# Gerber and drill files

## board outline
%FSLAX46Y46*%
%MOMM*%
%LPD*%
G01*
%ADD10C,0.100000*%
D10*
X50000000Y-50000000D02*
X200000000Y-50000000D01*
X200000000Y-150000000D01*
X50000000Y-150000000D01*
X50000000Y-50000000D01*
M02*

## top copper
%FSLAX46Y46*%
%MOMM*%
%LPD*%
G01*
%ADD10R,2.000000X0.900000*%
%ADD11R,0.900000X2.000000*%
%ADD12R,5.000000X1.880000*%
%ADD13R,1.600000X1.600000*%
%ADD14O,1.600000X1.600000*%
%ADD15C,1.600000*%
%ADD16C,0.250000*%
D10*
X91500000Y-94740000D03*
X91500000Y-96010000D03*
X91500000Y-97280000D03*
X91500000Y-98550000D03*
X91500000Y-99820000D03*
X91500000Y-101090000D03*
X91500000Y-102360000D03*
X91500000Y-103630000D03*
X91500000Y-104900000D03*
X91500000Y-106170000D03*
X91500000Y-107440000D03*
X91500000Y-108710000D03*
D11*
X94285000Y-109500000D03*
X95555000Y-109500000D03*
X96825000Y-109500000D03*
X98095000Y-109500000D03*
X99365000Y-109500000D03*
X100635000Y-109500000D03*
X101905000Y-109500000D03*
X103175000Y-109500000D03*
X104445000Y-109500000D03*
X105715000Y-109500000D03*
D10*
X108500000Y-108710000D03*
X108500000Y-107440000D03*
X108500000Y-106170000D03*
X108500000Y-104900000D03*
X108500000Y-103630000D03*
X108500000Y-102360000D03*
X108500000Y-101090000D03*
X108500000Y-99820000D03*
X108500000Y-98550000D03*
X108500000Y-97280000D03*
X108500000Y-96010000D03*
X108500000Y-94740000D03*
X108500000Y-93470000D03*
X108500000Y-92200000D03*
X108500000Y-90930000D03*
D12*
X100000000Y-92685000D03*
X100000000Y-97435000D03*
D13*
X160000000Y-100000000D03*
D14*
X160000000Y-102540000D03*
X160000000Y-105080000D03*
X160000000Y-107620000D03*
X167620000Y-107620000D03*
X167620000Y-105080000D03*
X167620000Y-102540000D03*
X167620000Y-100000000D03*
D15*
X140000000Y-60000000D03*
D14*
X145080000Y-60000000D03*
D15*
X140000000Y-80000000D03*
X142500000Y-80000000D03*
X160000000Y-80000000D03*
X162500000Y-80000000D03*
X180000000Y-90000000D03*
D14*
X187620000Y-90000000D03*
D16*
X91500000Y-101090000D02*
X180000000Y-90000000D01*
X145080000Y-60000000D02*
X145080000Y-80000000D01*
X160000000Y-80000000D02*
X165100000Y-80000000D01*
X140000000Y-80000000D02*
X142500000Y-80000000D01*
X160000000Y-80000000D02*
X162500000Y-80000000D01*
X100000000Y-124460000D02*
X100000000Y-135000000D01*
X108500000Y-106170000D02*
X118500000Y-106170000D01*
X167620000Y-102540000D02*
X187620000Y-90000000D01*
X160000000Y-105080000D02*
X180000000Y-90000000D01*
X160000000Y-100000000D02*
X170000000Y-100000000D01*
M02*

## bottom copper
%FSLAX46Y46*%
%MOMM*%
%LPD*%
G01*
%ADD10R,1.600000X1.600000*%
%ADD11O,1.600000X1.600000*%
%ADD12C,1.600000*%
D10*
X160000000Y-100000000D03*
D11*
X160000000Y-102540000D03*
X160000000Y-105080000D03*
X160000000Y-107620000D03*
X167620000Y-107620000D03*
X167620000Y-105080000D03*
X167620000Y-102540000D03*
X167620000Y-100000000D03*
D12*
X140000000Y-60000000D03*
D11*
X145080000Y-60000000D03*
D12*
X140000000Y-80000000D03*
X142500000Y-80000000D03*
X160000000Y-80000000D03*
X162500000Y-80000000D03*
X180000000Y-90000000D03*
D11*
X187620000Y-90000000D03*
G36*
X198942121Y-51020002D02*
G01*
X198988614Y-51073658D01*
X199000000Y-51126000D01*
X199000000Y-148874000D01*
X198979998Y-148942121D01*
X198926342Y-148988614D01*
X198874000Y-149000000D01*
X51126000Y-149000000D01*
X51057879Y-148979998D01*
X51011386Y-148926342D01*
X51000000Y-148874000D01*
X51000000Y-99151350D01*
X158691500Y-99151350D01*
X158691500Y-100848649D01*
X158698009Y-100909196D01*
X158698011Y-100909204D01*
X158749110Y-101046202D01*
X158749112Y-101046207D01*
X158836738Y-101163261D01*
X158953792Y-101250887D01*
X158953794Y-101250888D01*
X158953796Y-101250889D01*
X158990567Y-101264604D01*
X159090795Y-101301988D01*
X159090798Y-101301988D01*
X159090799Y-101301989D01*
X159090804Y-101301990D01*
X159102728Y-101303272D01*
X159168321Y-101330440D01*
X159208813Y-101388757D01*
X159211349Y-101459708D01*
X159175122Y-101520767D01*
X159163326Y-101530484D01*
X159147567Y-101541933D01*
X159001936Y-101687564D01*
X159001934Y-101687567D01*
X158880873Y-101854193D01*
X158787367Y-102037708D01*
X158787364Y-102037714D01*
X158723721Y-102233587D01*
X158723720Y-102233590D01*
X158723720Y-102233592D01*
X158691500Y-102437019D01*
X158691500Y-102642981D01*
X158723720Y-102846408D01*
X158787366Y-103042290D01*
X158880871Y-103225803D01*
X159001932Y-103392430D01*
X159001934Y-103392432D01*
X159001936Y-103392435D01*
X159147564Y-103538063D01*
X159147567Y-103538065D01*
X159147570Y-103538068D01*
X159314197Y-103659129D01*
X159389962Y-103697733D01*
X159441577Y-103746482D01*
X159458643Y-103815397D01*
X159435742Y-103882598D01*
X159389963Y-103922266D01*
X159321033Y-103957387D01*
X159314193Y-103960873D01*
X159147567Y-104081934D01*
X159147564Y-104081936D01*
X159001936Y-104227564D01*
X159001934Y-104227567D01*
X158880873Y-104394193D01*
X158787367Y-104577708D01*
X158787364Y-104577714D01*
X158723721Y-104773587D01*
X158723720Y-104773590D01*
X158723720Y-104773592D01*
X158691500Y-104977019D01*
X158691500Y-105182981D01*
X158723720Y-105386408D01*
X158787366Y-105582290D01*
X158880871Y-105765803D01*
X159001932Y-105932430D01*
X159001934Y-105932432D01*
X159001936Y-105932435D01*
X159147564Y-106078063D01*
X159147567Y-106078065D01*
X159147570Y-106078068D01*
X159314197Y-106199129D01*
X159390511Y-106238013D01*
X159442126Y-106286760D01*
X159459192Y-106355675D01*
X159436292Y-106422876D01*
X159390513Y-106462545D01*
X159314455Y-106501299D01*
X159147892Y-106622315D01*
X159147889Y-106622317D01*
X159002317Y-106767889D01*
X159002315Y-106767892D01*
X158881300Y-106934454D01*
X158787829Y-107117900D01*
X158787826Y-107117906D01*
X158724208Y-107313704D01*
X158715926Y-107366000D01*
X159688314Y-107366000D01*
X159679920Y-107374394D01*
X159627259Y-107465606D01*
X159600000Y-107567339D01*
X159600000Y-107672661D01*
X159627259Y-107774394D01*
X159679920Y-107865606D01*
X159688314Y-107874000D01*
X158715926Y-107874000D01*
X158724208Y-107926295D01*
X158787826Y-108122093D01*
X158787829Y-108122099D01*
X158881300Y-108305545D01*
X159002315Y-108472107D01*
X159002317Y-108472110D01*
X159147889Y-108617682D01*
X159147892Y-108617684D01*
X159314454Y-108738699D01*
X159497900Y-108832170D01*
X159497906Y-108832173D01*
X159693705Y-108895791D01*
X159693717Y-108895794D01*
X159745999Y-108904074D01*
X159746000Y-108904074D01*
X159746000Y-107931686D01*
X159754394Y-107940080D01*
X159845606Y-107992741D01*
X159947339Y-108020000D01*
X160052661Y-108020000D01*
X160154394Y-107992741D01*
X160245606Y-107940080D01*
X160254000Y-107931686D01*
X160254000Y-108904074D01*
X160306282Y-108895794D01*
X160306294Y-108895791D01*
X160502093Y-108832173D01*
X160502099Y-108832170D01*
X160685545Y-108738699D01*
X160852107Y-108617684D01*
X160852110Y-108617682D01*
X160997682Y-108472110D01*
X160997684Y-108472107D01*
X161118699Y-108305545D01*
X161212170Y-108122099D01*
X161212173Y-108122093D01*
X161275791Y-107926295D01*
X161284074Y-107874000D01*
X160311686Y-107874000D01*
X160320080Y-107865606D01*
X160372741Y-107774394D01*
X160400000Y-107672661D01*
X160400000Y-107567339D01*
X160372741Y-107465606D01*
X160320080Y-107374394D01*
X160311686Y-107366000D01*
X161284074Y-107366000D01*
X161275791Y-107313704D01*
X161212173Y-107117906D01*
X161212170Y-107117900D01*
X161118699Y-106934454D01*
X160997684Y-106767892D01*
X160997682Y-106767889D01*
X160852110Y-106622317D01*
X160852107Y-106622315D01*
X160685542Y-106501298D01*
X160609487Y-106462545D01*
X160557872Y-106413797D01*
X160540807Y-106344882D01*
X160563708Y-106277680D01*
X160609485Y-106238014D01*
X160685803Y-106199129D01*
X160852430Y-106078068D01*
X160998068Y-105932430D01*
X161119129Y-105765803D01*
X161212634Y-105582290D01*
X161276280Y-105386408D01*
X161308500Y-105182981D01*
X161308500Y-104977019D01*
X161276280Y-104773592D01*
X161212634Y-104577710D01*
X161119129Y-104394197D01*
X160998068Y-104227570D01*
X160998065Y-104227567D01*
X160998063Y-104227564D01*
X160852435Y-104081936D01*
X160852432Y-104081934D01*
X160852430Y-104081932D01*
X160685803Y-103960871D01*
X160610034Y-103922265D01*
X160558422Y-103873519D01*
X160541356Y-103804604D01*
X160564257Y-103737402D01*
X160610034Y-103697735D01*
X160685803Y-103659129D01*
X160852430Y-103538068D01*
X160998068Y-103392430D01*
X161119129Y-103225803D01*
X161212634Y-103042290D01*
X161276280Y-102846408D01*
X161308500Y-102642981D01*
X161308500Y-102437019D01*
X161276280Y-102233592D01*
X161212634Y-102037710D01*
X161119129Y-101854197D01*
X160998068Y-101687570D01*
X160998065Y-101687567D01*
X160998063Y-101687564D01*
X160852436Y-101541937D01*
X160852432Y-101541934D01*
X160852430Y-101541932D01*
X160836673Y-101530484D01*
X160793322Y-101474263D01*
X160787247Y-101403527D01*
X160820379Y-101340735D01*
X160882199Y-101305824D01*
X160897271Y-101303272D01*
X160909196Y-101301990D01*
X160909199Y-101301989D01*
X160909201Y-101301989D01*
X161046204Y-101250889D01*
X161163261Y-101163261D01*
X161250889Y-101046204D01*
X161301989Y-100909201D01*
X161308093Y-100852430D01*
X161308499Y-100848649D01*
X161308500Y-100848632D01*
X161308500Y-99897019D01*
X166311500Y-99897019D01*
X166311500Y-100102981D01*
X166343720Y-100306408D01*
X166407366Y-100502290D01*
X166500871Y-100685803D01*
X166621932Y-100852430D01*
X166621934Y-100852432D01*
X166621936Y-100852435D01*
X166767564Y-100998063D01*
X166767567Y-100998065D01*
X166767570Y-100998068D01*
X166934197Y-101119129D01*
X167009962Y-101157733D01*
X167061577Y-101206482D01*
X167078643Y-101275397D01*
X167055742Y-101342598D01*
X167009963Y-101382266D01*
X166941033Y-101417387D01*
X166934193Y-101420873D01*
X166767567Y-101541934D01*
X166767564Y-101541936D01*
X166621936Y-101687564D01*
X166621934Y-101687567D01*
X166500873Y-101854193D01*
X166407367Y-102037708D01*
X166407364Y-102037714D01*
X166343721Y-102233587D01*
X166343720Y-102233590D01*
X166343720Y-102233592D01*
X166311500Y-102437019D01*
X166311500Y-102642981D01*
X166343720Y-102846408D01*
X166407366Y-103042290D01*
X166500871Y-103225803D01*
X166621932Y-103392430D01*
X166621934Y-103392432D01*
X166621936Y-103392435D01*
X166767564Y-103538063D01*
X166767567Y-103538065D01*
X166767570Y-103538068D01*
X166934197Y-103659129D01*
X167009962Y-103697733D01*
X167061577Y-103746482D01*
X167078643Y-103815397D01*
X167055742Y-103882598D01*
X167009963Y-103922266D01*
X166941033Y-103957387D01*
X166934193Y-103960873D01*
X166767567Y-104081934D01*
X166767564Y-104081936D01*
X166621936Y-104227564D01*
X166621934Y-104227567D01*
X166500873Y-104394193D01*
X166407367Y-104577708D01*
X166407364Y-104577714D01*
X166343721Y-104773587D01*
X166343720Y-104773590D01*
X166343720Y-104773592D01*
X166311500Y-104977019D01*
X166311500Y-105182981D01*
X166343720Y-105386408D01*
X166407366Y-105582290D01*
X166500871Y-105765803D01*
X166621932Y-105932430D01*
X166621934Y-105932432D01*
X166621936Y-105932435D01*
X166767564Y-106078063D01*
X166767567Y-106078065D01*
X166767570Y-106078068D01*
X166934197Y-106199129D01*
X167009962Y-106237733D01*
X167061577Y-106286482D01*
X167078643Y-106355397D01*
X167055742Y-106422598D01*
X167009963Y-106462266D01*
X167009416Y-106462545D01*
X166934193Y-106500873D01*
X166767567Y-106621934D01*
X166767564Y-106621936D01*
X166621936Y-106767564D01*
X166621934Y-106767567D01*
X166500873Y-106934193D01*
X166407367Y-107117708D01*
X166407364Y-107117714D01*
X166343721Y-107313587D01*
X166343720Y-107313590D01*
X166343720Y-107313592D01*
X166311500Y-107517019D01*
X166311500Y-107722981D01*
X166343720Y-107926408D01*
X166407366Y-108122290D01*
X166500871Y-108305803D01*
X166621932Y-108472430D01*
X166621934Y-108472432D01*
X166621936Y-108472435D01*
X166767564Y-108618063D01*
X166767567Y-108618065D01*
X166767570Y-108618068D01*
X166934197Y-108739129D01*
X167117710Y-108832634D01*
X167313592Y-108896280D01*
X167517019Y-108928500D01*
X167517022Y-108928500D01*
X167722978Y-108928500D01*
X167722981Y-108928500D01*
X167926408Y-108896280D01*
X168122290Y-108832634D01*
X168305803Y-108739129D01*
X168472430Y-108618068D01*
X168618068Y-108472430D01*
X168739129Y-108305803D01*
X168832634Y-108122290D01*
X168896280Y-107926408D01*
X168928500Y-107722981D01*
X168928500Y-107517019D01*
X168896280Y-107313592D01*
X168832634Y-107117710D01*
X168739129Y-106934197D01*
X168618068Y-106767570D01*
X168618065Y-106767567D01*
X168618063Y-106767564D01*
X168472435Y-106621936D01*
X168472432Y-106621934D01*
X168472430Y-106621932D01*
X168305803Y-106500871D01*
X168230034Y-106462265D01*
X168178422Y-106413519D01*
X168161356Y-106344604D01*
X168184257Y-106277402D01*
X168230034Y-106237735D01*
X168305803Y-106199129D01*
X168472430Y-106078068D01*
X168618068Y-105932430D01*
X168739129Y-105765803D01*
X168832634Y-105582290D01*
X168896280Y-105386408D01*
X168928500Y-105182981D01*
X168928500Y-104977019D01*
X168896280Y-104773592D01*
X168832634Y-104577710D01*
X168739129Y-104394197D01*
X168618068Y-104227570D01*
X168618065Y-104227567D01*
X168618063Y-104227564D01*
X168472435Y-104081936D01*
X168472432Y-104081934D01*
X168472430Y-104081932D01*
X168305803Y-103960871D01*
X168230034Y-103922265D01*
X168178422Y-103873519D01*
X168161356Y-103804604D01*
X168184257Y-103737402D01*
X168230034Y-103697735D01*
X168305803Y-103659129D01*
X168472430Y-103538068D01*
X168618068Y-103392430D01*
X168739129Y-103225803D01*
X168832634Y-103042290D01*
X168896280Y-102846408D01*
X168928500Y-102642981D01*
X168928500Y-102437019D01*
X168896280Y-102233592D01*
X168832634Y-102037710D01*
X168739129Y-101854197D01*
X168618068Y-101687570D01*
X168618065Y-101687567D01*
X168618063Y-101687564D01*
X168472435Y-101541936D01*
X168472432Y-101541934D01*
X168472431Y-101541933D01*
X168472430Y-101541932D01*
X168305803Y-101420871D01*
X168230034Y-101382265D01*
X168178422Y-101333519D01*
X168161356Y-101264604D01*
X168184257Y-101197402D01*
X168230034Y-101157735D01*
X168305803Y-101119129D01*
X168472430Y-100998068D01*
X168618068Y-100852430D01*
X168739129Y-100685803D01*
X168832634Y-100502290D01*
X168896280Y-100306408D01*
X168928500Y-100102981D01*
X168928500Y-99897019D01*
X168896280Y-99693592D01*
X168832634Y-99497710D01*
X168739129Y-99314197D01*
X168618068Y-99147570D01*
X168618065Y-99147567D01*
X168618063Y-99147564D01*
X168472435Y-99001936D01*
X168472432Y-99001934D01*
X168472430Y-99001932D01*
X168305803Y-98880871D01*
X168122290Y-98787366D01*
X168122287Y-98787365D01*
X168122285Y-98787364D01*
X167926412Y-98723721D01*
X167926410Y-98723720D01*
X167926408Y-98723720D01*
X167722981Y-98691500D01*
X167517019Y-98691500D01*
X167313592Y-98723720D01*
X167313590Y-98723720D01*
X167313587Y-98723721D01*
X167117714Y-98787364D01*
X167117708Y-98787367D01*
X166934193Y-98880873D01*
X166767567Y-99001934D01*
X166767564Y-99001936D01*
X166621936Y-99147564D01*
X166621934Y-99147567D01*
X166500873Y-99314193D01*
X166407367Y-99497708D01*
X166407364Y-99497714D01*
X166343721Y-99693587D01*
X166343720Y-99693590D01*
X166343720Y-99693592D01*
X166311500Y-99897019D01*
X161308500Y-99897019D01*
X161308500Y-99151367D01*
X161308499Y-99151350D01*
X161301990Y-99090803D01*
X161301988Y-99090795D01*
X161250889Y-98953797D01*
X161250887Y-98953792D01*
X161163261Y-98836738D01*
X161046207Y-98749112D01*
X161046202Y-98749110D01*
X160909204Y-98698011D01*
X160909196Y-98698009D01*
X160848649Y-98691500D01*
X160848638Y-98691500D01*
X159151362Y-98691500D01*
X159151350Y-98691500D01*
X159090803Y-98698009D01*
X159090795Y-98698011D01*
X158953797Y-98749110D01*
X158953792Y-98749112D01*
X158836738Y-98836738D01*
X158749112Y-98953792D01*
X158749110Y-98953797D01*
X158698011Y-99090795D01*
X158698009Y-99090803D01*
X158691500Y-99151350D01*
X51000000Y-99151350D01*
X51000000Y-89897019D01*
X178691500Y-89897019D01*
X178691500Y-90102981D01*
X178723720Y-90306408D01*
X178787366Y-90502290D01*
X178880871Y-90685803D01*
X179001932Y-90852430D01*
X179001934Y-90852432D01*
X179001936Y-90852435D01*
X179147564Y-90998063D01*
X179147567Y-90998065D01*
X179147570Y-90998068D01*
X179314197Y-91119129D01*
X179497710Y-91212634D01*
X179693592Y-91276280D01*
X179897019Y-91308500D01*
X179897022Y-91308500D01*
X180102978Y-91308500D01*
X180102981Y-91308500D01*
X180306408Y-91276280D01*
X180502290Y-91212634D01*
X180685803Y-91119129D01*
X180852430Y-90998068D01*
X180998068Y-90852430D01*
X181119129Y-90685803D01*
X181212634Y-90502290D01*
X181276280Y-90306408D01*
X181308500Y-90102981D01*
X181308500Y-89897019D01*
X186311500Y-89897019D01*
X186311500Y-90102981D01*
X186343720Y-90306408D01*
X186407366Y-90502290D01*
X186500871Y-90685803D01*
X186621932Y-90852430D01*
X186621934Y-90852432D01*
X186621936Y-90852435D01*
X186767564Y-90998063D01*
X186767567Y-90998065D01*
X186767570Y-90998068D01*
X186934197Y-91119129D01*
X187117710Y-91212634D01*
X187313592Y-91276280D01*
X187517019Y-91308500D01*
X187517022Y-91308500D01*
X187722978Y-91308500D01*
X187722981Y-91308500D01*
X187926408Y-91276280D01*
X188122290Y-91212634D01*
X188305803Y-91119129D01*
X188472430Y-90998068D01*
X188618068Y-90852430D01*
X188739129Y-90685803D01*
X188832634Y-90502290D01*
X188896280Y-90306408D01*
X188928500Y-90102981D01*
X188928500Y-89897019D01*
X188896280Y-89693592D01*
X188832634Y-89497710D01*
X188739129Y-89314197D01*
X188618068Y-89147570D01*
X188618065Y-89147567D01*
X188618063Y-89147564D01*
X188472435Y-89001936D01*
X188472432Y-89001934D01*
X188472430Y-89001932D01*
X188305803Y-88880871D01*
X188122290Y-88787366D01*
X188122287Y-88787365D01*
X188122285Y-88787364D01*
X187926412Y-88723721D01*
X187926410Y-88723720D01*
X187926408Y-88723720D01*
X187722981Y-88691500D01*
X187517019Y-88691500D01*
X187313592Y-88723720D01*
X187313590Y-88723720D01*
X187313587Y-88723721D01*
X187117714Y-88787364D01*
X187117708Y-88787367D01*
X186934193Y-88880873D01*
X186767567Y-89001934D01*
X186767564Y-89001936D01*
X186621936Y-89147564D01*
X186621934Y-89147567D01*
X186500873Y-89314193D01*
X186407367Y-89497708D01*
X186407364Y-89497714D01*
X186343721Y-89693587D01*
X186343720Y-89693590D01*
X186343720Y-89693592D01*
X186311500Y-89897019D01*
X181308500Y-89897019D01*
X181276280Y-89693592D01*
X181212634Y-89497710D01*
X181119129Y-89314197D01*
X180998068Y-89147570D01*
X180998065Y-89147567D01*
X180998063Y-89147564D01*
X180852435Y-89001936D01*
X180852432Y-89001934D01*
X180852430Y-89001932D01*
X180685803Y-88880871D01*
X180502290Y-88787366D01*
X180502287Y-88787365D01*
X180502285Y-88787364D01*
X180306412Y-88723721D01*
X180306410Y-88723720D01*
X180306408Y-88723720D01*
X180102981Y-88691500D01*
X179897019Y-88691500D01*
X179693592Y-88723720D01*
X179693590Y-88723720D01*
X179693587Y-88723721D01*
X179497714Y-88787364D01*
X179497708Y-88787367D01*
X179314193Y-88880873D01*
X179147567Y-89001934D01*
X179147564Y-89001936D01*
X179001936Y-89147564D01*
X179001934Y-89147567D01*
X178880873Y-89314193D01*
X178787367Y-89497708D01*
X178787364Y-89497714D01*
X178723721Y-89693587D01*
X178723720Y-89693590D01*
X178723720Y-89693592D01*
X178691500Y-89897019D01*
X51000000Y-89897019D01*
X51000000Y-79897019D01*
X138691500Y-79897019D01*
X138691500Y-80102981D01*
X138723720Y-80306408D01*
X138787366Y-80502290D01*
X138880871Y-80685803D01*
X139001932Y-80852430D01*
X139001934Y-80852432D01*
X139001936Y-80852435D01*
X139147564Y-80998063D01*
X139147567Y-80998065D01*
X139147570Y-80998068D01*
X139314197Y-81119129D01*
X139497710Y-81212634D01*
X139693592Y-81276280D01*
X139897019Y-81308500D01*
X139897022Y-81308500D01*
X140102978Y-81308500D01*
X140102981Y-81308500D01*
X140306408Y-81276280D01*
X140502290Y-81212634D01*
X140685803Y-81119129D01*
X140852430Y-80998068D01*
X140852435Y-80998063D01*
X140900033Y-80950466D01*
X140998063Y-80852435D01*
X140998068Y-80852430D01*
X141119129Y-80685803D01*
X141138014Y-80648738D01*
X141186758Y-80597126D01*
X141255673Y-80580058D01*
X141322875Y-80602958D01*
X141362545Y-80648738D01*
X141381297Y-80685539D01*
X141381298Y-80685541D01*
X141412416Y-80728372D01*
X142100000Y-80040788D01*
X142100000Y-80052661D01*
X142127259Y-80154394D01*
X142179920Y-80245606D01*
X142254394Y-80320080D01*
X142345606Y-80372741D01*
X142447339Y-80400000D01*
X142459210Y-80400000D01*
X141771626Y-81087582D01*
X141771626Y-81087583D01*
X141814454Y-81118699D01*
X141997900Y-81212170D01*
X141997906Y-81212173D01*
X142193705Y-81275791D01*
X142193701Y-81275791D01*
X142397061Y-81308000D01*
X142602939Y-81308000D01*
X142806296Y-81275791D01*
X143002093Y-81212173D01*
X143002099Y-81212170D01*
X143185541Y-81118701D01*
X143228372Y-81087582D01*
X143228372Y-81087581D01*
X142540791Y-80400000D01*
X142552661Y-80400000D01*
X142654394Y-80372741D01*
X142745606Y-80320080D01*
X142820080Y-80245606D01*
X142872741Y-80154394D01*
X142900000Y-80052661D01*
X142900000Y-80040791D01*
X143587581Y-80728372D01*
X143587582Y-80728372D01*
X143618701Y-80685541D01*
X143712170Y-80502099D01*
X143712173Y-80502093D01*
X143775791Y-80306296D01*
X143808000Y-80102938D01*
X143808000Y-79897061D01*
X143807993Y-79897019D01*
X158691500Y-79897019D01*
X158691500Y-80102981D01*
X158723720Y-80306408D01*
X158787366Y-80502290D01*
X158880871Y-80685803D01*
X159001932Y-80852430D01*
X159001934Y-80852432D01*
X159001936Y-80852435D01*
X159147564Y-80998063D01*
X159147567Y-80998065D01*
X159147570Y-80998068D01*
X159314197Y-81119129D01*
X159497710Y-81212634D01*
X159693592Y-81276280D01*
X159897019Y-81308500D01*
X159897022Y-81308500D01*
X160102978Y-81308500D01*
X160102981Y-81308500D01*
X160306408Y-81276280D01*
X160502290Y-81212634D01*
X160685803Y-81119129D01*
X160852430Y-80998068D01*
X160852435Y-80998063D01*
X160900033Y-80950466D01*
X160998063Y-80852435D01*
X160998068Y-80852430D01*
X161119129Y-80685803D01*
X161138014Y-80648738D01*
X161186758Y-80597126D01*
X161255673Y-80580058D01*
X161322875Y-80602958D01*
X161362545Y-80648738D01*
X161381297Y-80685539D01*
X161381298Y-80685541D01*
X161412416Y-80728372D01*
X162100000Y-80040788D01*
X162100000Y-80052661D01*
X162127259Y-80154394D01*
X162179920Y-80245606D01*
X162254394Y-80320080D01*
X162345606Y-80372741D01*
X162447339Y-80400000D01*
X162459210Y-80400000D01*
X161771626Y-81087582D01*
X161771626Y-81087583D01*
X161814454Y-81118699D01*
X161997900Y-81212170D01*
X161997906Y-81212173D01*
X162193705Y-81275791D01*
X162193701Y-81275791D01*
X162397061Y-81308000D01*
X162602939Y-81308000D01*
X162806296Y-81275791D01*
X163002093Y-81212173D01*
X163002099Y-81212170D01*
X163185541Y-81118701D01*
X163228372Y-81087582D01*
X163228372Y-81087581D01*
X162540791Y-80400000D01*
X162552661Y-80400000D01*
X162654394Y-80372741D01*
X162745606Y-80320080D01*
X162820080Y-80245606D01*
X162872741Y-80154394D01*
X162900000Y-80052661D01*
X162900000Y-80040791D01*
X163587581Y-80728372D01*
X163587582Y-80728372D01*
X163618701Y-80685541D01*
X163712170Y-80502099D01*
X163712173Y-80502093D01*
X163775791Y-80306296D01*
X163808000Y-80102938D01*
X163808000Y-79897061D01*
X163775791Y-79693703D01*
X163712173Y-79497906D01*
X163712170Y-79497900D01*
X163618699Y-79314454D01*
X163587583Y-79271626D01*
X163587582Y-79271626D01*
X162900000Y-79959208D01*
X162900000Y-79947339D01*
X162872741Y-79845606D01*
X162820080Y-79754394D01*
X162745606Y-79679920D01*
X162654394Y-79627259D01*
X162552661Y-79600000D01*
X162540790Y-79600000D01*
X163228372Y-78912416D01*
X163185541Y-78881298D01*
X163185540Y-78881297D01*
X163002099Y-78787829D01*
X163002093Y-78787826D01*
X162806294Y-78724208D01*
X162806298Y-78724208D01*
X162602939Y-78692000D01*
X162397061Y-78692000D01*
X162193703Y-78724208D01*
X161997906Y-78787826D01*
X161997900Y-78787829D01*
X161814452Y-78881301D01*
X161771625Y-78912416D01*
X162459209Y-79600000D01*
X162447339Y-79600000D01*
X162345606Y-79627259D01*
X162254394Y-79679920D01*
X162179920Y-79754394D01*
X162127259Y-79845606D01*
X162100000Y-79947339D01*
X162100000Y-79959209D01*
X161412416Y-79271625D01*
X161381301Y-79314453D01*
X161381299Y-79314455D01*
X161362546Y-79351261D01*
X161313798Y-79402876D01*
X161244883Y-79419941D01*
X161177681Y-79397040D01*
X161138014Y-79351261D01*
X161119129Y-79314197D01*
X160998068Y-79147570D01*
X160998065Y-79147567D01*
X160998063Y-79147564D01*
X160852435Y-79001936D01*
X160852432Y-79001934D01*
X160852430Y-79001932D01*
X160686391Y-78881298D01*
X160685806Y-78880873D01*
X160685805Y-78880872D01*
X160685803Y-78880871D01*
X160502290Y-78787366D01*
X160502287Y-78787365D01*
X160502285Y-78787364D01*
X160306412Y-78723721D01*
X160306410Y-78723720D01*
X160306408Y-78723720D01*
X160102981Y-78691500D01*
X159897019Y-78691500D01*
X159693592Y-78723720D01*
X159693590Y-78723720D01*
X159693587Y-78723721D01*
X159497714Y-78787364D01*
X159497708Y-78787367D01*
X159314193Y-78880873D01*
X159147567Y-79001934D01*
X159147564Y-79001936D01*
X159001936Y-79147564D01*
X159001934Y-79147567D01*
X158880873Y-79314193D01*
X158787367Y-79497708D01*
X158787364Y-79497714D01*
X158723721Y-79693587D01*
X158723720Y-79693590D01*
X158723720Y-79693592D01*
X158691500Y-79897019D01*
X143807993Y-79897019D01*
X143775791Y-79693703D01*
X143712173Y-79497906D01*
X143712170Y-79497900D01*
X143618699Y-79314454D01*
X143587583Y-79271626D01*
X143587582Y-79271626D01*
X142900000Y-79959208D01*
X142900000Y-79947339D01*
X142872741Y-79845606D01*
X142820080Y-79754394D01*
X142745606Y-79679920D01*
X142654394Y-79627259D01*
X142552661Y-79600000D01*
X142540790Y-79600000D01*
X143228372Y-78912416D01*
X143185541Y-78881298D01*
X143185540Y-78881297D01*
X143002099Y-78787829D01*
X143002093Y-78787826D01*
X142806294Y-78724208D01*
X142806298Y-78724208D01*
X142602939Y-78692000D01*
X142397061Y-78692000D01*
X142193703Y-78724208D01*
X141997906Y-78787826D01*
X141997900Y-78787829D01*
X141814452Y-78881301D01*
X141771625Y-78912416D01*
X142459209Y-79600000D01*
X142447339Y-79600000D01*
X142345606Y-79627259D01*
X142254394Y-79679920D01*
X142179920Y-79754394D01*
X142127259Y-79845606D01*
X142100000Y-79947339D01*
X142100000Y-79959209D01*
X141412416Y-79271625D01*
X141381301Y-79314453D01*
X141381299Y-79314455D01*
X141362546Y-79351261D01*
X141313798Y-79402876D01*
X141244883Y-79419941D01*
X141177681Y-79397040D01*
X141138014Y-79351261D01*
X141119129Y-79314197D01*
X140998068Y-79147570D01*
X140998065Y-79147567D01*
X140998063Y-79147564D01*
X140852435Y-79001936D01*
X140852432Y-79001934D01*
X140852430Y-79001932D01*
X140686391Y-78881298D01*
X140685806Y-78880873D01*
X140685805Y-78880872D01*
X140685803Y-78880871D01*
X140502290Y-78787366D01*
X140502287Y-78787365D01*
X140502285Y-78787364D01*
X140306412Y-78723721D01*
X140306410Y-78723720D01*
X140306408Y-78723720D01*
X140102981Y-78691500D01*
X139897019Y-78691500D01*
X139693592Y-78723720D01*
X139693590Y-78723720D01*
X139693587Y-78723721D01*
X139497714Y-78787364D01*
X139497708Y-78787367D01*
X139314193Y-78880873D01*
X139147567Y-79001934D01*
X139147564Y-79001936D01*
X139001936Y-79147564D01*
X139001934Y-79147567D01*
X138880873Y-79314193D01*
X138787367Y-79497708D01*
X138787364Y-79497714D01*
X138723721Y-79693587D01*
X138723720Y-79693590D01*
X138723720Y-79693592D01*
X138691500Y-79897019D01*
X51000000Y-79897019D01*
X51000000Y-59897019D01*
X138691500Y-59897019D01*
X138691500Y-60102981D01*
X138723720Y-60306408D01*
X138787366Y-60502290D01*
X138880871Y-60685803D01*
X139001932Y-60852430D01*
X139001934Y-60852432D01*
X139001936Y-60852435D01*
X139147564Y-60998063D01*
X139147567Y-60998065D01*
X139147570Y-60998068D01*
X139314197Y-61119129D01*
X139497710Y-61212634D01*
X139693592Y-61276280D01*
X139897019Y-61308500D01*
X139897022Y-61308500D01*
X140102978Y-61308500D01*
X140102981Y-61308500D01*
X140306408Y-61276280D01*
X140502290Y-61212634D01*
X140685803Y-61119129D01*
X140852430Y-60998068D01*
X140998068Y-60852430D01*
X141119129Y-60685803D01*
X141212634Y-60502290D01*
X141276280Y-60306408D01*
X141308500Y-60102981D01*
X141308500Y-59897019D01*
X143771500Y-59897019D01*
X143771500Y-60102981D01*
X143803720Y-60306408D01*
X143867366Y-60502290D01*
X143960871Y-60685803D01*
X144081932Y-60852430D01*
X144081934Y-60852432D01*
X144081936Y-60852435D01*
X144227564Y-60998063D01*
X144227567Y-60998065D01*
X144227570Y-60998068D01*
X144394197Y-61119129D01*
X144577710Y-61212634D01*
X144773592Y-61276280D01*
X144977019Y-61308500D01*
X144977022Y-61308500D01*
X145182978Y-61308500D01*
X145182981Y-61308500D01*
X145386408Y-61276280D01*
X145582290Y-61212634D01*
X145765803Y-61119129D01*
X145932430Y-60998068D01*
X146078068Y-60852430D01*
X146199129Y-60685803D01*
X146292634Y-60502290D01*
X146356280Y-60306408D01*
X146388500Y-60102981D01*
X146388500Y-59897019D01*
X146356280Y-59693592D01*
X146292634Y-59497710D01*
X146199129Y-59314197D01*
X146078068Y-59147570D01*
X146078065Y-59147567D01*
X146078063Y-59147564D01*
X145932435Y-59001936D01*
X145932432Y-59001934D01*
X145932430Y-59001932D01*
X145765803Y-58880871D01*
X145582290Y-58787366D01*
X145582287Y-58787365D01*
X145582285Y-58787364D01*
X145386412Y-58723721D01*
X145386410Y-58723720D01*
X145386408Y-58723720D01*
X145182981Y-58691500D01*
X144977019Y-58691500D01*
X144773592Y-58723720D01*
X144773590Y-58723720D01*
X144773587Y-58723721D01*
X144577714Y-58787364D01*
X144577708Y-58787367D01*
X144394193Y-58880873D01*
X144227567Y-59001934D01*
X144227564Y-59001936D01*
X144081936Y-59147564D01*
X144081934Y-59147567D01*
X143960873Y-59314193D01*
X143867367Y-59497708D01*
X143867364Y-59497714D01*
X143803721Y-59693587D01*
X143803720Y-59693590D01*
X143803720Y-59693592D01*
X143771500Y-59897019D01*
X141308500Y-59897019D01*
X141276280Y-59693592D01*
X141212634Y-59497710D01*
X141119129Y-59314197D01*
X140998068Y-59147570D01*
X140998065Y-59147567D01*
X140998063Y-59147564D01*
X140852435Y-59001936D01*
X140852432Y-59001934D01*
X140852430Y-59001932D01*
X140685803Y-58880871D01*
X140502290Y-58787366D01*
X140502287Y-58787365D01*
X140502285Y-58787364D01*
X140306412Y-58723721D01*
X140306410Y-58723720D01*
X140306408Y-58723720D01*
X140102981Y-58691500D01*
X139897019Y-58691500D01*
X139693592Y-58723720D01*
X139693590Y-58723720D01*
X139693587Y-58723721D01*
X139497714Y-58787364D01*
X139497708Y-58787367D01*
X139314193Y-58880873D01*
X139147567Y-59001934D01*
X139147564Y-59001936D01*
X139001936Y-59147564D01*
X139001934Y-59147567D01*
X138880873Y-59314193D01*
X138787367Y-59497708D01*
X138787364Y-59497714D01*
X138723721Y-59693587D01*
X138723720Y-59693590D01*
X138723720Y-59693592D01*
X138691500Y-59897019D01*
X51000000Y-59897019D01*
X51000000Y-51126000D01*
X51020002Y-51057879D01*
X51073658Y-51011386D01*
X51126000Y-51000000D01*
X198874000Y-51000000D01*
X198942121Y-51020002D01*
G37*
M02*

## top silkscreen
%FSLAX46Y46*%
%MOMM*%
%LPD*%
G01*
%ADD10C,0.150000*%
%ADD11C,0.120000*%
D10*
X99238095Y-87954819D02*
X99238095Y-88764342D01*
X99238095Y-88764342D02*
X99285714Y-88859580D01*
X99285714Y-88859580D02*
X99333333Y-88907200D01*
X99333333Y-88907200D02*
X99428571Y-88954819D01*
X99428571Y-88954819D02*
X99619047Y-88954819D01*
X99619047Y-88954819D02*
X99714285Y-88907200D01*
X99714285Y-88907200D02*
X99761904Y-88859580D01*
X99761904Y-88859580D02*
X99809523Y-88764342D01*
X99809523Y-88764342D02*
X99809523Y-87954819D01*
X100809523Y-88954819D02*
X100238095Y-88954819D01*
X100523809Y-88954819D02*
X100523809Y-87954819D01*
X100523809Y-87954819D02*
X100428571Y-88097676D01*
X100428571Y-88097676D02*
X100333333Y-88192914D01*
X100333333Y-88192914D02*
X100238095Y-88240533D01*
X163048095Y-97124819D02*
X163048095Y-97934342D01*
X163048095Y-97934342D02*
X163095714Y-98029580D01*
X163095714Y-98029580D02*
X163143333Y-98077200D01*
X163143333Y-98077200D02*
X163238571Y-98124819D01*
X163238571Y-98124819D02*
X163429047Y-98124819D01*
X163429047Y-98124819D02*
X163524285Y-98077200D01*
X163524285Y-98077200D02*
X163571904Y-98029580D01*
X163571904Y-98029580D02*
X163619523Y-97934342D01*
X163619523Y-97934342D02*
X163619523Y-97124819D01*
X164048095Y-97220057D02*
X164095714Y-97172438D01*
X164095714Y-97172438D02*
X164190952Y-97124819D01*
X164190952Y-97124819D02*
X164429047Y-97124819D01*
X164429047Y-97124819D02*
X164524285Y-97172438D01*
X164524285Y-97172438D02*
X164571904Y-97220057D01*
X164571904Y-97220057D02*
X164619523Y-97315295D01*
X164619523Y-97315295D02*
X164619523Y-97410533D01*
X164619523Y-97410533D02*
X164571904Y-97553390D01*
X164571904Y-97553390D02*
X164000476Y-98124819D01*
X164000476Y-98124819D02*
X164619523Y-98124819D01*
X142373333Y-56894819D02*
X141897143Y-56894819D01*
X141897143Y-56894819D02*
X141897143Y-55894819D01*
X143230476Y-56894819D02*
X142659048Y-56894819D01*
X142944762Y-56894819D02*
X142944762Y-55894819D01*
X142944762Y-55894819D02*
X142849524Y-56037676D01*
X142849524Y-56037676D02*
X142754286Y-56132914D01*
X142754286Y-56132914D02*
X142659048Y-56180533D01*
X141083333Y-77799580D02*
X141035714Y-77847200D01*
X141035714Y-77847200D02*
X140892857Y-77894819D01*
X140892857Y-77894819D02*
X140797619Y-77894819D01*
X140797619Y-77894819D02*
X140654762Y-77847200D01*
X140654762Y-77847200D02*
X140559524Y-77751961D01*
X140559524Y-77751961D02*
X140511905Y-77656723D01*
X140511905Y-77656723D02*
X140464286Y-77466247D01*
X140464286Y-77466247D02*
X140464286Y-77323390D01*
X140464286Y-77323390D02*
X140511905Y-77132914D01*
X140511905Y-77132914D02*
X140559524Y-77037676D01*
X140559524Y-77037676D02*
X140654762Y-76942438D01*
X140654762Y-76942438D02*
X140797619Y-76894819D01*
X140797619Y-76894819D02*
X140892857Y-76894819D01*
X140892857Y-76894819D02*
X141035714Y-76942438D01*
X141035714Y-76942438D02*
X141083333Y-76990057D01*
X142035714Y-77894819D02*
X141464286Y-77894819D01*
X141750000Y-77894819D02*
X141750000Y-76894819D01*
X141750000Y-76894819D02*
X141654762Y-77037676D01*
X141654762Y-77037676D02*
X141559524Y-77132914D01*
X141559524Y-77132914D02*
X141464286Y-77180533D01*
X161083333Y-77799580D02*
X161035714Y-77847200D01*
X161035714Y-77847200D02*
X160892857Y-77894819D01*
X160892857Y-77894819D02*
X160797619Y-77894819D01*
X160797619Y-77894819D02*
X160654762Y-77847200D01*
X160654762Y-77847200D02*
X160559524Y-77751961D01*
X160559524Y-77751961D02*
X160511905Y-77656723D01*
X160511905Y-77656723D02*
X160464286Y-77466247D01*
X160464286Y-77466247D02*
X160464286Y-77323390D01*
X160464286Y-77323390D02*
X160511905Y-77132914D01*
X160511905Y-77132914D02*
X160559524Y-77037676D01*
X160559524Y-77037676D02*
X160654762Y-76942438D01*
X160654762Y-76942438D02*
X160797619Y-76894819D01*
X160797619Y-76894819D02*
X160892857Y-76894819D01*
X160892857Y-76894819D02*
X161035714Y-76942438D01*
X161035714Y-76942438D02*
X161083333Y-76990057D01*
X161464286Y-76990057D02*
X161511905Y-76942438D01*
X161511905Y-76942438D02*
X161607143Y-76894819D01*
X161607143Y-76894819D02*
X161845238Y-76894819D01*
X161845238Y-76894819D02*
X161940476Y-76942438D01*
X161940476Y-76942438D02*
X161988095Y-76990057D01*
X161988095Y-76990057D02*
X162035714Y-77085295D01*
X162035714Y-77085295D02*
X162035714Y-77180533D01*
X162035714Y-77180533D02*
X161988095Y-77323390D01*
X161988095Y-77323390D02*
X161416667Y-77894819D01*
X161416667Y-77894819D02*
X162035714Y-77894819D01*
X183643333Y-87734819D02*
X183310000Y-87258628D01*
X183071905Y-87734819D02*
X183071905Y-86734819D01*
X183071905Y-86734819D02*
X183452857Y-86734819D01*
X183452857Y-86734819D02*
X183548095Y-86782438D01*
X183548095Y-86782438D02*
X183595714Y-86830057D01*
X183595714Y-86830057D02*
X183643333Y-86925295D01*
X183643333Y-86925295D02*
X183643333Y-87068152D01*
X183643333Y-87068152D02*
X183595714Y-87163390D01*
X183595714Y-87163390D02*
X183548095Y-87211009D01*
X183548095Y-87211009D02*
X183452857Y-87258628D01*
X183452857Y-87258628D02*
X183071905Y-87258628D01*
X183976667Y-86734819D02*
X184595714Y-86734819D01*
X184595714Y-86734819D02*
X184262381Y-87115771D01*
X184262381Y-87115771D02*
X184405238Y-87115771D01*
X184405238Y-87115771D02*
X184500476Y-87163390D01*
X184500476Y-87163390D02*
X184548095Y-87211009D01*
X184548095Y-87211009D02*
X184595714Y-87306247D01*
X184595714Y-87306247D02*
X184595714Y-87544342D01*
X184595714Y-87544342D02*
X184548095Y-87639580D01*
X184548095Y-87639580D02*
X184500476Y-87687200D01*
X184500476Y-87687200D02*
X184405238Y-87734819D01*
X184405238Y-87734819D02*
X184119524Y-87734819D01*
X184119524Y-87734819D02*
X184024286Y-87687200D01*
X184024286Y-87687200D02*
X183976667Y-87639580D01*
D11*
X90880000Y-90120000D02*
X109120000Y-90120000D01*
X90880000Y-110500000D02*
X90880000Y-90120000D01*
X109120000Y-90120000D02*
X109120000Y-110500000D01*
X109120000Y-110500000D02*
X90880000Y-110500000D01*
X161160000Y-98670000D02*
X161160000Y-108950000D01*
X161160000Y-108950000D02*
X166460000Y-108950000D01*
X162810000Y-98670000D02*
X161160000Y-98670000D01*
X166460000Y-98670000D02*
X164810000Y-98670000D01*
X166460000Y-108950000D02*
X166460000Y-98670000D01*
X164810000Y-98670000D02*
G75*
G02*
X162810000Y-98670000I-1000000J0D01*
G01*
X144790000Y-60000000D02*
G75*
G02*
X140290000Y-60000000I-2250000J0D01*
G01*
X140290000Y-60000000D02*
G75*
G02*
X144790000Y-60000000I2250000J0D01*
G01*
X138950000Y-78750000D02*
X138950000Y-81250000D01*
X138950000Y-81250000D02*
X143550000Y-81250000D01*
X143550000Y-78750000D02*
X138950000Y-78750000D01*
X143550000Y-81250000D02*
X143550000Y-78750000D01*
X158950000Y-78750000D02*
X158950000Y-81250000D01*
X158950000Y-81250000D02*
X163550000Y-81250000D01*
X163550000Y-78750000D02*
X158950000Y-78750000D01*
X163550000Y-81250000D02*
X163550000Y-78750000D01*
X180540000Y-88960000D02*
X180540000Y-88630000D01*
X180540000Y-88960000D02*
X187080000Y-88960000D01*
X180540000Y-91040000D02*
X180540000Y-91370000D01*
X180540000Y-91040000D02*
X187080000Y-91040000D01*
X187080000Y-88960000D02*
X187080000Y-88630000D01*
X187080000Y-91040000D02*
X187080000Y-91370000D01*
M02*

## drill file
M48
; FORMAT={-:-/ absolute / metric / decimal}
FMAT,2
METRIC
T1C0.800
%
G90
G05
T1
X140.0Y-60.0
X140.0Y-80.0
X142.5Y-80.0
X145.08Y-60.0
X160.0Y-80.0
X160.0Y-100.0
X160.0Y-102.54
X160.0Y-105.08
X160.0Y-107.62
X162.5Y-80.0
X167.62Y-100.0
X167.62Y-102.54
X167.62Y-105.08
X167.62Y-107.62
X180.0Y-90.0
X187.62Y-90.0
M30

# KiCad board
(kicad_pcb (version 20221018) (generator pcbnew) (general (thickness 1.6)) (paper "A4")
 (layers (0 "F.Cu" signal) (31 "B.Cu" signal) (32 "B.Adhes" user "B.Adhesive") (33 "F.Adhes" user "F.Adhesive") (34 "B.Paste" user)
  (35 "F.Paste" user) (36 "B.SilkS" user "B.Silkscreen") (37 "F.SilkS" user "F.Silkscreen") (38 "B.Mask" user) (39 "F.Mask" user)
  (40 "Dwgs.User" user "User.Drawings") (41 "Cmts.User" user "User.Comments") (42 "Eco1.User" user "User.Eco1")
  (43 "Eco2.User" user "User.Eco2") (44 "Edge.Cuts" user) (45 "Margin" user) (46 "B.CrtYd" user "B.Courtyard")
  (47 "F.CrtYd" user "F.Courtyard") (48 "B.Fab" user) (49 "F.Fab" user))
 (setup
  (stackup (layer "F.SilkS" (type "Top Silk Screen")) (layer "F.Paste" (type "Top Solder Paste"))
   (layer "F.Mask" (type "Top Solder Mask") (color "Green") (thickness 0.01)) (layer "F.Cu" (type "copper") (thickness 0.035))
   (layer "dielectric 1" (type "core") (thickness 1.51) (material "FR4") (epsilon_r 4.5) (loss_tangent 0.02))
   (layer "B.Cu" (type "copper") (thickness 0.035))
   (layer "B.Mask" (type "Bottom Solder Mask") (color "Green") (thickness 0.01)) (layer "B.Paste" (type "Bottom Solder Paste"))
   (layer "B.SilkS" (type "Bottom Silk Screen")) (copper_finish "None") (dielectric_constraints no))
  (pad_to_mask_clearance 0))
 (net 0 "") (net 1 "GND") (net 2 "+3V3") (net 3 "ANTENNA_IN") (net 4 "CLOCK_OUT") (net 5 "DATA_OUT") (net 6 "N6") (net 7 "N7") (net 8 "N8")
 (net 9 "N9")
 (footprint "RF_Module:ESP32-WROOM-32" (layer "F.Cu") (at 100 100)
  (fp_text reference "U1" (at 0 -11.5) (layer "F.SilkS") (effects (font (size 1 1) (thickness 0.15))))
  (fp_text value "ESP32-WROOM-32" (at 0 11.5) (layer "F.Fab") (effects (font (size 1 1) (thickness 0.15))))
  (fp_line (start -9.12 -9.88) (end 9.12 -9.88) (stroke (width 0.12) (type solid)) (layer "F.SilkS"))
  (fp_line (start -9.12 10.5) (end -9.12 -9.88) (stroke (width 0.12) (type solid)) (layer "F.SilkS"))
  (fp_line (start 9.12 -9.88) (end 9.12 10.5) (stroke (width 0.12) (type solid)) (layer "F.SilkS"))
  (fp_line (start 9.12 10.5) (end -9.12 10.5) (stroke (width 0.12) (type solid)) (layer "F.SilkS"))
  (pad "1" smd rect (at -8.5 -5.26) (size 2 0.9) (layers "F.Cu" "F.Paste" "F.Mask") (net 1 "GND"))
  (pad "2" smd rect (at -8.5 -3.99) (size 2 0.9) (layers "F.Cu" "F.Paste" "F.Mask") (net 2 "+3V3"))
  (pad "3" smd rect (at -8.5 -2.72) (size 2 0.9) (layers "F.Cu" "F.Paste" "F.Mask"))
  (pad "4" smd rect (at -8.5 -1.45) (size 2 0.9) (layers "F.Cu" "F.Paste" "F.Mask"))
  (pad "5" smd rect (at -8.5 -0.18) (size 2 0.9) (layers "F.Cu" "F.Paste" "F.Mask"))
  (pad "6" smd rect (at -8.5 1.09) (size 2 0.9) (layers "F.Cu" "F.Paste" "F.Mask") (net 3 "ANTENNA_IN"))
  (pad "7" smd rect (at -8.5 2.36) (size 2 0.9) (layers "F.Cu" "F.Paste" "F.Mask"))
  (pad "8" smd rect (at -8.5 3.63) (size 2 0.9) (layers "F.Cu" "F.Paste" "F.Mask"))
  (pad "9" smd rect (at -8.5 4.9) (size 2 0.9) (layers "F.Cu" "F.Paste" "F.Mask"))
  (pad "10" smd rect (at -8.5 6.17) (size 2 0.9) (layers "F.Cu" "F.Paste" "F.Mask") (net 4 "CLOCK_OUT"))
  (pad "11" smd rect (at -8.5 7.44) (size 2 0.9) (layers "F.Cu" "F.Paste" "F.Mask"))
  (pad "12" smd rect (at -8.5 8.71) (size 2 0.9) (layers "F.Cu" "F.Paste" "F.Mask"))
  (pad "13" smd rect (at -5.715 9.5) (size 0.9 2) (layers "F.Cu" "F.Paste" "F.Mask"))
  (pad "14" smd rect (at -4.445 9.5) (size 0.9 2) (layers "F.Cu" "F.Paste" "F.Mask"))
  (pad "15" smd rect (at -3.175 9.5) (size 0.9 2) (layers "F.Cu" "F.Paste" "F.Mask") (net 1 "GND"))
  (pad "16" smd rect (at -1.905 9.5) (size 0.9 2) (layers "F.Cu" "F.Paste" "F.Mask"))
  (pad "17" smd rect (at -0.635 9.5) (size 0.9 2) (layers "F.Cu" "F.Paste" "F.Mask"))
  (pad "18" smd rect (at 0.635 9.5) (size 0.9 2) (layers "F.Cu" "F.Paste" "F.Mask"))
  (pad "19" smd rect (at 1.905 9.5) (size 0.9 2) (layers "F.Cu" "F.Paste" "F.Mask"))
  (pad "20" smd rect (at 3.175 9.5) (size 0.9 2) (layers "F.Cu" "F.Paste" "F.Mask"))
  (pad "21" smd rect (at 4.445 9.5) (size 0.9 2) (layers "F.Cu" "F.Paste" "F.Mask"))
  (pad "22" smd rect (at 5.715 9.5) (size 0.9 2) (layers "F.Cu" "F.Paste" "F.Mask"))
  (pad "23" smd rect (at 8.5 8.71) (size 2 0.9) (layers "F.Cu" "F.Paste" "F.Mask"))
  (pad "24" smd rect (at 8.5 7.44) (size 2 0.9) (layers "F.Cu" "F.Paste" "F.Mask"))
  (pad "25" smd rect (at 8.5 6.17) (size 2 0.9) (layers "F.Cu" "F.Paste" "F.Mask"))
  (pad "26" smd rect (at 8.5 4.9) (size 2 0.9) (layers "F.Cu" "F.Paste" "F.Mask"))
  (pad "27" smd rect (at 8.5 3.63) (size 2 0.9) (layers "F.Cu" "F.Paste" "F.Mask"))
  (pad "28" smd rect (at 8.5 2.36) (size 2 0.9) (layers "F.Cu" "F.Paste" "F.Mask"))
  (pad "29" smd rect (at 8.5 1.09) (size 2 0.9) (layers "F.Cu" "F.Paste" "F.Mask"))
  (pad "30" smd rect (at 8.5 -0.18) (size 2 0.9) (layers "F.Cu" "F.Paste" "F.Mask"))
  (pad "31" smd rect (at 8.5 -1.45) (size 2 0.9) (layers "F.Cu" "F.Paste" "F.Mask"))
  (pad "32" smd rect (at 8.5 -2.72) (size 2 0.9) (layers "F.Cu" "F.Paste" "F.Mask"))
  (pad "33" smd rect (at 8.5 -3.99) (size 2 0.9) (layers "F.Cu" "F.Paste" "F.Mask"))
  (pad "34" smd rect (at 8.5 -5.26) (size 2 0.9) (layers "F.Cu" "F.Paste" "F.Mask"))
  (pad "35" smd rect (at 8.5 -6.53) (size 2 0.9) (layers "F.Cu" "F.Paste" "F.Mask"))
  (pad "36" smd rect (at 8.5 -7.8) (size 2 0.9) (layers "F.Cu" "F.Paste" "F.Mask"))
  (pad "37" smd rect (at 8.5 -9.07) (size 2 0.9) (layers "F.Cu" "F.Paste" "F.Mask"))
  (pad "38" smd rect (at 0 -7.315) (size 5 1.88) (layers "F.Cu" "F.Paste" "F.Mask") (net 1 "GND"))
  (pad "39" smd rect (at 0 -2.565) (size 5 1.88) (layers "F.Cu" "F.Paste" "F.Mask") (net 1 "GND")))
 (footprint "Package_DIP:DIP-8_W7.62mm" (layer "F.Cu") (at 160 100)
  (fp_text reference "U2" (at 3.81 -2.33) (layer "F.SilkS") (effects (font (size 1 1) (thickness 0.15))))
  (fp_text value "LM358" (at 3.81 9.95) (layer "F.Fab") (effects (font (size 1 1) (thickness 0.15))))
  (fp_line (start 1.16 -1.33) (end 1.16 8.95) (stroke (width 0.12) (type solid)) (layer "F.SilkS"))
  (fp_line (start 1.16 8.95) (end 6.46 8.95) (stroke (width 0.12) (type solid)) (layer "F.SilkS"))
  (fp_line (start 2.81 -1.33) (end 1.16 -1.33) (stroke (width 0.12) (type solid)) (layer "F.SilkS"))
  (fp_line (start 6.46 -1.33) (end 4.81 -1.33) (stroke (width 0.12) (type solid)) (layer "F.SilkS"))
  (fp_line (start 6.46 8.95) (end 6.46 -1.33) (stroke (width 0.12) (type solid)) (layer "F.SilkS"))
  (fp_arc (start 4.81 -1.33) (mid 3.81 -0.33) (end 2.81 -1.33) (stroke (width 0.12) (type solid)) (layer "F.SilkS"))
  (pad "1" thru_hole rect (at 0 0) (size 1.6 1.6) (drill 0.8) (layers "*.Cu" "*.Mask") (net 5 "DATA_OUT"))
  (pad "2" thru_hole oval (at 0 2.54) (size 1.6 1.6) (drill 0.8) (layers "*.Cu" "*.Mask") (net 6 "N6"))
  (pad "3" thru_hole oval (at 0 5.08) (size 1.6 1.6) (drill 0.8) (layers "*.Cu" "*.Mask") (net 3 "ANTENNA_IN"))
  (pad "4" thru_hole oval (at 0 7.62) (size 1.6 1.6) (drill 0.8) (layers "*.Cu" "*.Mask") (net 1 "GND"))
  (pad "5" thru_hole oval (at 7.62 7.62) (size 1.6 1.6) (drill 0.8) (layers "*.Cu" "*.Mask"))
  (pad "6" thru_hole oval (at 7.62 5.08) (size 1.6 1.6) (drill 0.8) (layers "*.Cu" "*.Mask"))
  (pad "7" thru_hole oval (at 7.62 2.54) (size 1.6 1.6) (drill 0.8) (layers "*.Cu" "*.Mask"))
  (pad "8" thru_hole oval (at 7.62 0) (size 1.6 1.6) (drill 0.8) (layers "*.Cu" "*.Mask") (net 2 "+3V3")))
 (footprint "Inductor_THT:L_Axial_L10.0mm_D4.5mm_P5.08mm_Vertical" (layer "F.Cu") (at 140 60)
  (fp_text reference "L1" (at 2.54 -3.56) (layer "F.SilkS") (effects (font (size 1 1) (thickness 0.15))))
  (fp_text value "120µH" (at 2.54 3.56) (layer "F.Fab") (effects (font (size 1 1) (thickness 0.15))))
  (fp_circle (center 2.54 0) (end 4.79 0) (stroke (width 0.12) (type solid)) (fill none) (layer "F.SilkS"))
  (pad "1" thru_hole circle (at 0 0) (size 1.6 1.6) (drill 0.8) (layers "*.Cu" "*.Mask") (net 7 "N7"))
  (pad "2" thru_hole oval (at 5.08 0) (size 1.6 1.6) (drill 0.8) (layers "*.Cu" "*.Mask") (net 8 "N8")))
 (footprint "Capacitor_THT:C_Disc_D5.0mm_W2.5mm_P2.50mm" (layer "F.Cu") (at 140 80)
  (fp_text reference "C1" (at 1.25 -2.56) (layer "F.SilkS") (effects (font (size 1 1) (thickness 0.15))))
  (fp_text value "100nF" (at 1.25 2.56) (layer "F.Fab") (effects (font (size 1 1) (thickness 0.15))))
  (fp_line (start -1.05 -1.25) (end -1.05 1.25) (stroke (width 0.12) (type solid)) (layer "F.SilkS"))
  (fp_line (start -1.05 1.25) (end 3.55 1.25) (stroke (width 0.12) (type solid)) (layer "F.SilkS"))
  (fp_line (start 3.55 -1.25) (end -1.05 -1.25) (stroke (width 0.12) (type solid)) (layer "F.SilkS"))
  (fp_line (start 3.55 1.25) (end 3.55 -1.25) (stroke (width 0.12) (type solid)) (layer "F.SilkS"))
  (pad "1" thru_hole circle (at 0 0) (size 1.6 1.6) (drill 0.8) (layers "*.Cu" "*.Mask") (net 8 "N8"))
  (pad "2" thru_hole circle (at 2.5 0) (size 1.6 1.6) (drill 0.8) (layers "*.Cu" "*.Mask") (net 1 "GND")))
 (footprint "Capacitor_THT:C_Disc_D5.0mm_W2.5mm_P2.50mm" (layer "F.Cu") (at 160 80)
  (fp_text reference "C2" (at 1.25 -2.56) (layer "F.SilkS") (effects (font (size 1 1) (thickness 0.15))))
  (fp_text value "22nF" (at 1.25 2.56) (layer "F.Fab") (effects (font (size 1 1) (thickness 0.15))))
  (fp_line (start -1.05 -1.25) (end -1.05 1.25) (stroke (width 0.12) (type solid)) (layer "F.SilkS"))
  (fp_line (start -1.05 1.25) (end 3.55 1.25) (stroke (width 0.12) (type solid)) (layer "F.SilkS"))
  (fp_line (start 3.55 -1.25) (end -1.05 -1.25) (stroke (width 0.12) (type solid)) (layer "F.SilkS"))
  (fp_line (start 3.55 1.25) (end 3.55 -1.25) (stroke (width 0.12) (type solid)) (layer "F.SilkS"))
  (pad "1" thru_hole circle (at 0 0) (size 1.6 1.6) (drill 0.8) (layers "*.Cu" "*.Mask") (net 8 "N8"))
  (pad "2" thru_hole circle (at 2.5 0) (size 1.6 1.6) (drill 0.8) (layers "*.Cu" "*.Mask") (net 1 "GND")))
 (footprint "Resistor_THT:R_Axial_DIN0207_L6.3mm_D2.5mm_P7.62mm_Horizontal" (layer "F.Cu") (at 180 90)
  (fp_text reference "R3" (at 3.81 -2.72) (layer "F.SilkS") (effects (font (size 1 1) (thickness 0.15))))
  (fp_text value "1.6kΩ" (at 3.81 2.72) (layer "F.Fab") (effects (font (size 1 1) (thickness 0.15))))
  (fp_line (start 0.54 -1.04) (end 0.54 -1.37) (stroke (width 0.12) (type solid)) (layer "F.SilkS"))
  (fp_line (start 0.54 -1.04) (end 7.08 -1.04) (stroke (width 0.12) (type solid)) (layer "F.SilkS"))
  (fp_line (start 0.54 1.04) (end 0.54 1.37) (stroke (width 0.12) (type solid)) (layer "F.SilkS"))
  (fp_line (start 0.54 1.04) (end 7.08 1.04) (stroke (width 0.12) (type solid)) (layer "F.SilkS"))
  (fp_line (start 7.08 -1.04) (end 7.08 -1.37) (stroke (width 0.12) (type solid)) (layer "F.SilkS"))
  (fp_line (start 7.08 1.04) (end 7.08 1.37) (stroke (width 0.12) (type solid)) (layer "F.SilkS"))
  (pad "1" thru_hole circle (at 0 0) (size 1.6 1.6) (drill 0.8) (layers "*.Cu" "*.Mask") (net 3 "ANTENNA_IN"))
  (pad "2" thru_hole oval (at 7.62 0) (size 1.6 1.6) (drill 0.8) (layers "*.Cu" "*.Mask") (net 6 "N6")))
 (gr_rect (start 50 50) (end 200 150) (stroke (width 0.1) (type solid)) (fill none) (layer "Edge.Cuts"))
 (segment (start 91.5 101.09) (end 180 90) (width 0.25) (layer "F.Cu") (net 3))
 (segment (start 145.08 60) (end 145.08 80) (width 0.25) (layer "F.Cu") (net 8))
 (segment (start 160 80) (end 165.1 80) (width 0.25) (layer "F.Cu") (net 8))
 (segment (start 140 80) (end 142.5 80) (width 0.25) (layer "F.Cu") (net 1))
 (segment (start 160 80) (end 162.5 80) (width 0.25) (layer "F.Cu") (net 1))
 (segment (start 100 124.46) (end 100 135) (width 0.25) (layer "F.Cu") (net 1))
 (segment (start 108.5 106.17) (end 118.5 106.17) (width 0.25) (layer "F.Cu") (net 4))
 (segment (start 167.62 102.54) (end 187.62 90) (width 0.25) (layer "F.Cu") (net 6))
 (segment (start 160 105.08) (end 180 90) (width 0.25) (layer "F.Cu") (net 3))
 (segment (start 160 100) (end 170 100) (width 0.25) (layer "F.Cu") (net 5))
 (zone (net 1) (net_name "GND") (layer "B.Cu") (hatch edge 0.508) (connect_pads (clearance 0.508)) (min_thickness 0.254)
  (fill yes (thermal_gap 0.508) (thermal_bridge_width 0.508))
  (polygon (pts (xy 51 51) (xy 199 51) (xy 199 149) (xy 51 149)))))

